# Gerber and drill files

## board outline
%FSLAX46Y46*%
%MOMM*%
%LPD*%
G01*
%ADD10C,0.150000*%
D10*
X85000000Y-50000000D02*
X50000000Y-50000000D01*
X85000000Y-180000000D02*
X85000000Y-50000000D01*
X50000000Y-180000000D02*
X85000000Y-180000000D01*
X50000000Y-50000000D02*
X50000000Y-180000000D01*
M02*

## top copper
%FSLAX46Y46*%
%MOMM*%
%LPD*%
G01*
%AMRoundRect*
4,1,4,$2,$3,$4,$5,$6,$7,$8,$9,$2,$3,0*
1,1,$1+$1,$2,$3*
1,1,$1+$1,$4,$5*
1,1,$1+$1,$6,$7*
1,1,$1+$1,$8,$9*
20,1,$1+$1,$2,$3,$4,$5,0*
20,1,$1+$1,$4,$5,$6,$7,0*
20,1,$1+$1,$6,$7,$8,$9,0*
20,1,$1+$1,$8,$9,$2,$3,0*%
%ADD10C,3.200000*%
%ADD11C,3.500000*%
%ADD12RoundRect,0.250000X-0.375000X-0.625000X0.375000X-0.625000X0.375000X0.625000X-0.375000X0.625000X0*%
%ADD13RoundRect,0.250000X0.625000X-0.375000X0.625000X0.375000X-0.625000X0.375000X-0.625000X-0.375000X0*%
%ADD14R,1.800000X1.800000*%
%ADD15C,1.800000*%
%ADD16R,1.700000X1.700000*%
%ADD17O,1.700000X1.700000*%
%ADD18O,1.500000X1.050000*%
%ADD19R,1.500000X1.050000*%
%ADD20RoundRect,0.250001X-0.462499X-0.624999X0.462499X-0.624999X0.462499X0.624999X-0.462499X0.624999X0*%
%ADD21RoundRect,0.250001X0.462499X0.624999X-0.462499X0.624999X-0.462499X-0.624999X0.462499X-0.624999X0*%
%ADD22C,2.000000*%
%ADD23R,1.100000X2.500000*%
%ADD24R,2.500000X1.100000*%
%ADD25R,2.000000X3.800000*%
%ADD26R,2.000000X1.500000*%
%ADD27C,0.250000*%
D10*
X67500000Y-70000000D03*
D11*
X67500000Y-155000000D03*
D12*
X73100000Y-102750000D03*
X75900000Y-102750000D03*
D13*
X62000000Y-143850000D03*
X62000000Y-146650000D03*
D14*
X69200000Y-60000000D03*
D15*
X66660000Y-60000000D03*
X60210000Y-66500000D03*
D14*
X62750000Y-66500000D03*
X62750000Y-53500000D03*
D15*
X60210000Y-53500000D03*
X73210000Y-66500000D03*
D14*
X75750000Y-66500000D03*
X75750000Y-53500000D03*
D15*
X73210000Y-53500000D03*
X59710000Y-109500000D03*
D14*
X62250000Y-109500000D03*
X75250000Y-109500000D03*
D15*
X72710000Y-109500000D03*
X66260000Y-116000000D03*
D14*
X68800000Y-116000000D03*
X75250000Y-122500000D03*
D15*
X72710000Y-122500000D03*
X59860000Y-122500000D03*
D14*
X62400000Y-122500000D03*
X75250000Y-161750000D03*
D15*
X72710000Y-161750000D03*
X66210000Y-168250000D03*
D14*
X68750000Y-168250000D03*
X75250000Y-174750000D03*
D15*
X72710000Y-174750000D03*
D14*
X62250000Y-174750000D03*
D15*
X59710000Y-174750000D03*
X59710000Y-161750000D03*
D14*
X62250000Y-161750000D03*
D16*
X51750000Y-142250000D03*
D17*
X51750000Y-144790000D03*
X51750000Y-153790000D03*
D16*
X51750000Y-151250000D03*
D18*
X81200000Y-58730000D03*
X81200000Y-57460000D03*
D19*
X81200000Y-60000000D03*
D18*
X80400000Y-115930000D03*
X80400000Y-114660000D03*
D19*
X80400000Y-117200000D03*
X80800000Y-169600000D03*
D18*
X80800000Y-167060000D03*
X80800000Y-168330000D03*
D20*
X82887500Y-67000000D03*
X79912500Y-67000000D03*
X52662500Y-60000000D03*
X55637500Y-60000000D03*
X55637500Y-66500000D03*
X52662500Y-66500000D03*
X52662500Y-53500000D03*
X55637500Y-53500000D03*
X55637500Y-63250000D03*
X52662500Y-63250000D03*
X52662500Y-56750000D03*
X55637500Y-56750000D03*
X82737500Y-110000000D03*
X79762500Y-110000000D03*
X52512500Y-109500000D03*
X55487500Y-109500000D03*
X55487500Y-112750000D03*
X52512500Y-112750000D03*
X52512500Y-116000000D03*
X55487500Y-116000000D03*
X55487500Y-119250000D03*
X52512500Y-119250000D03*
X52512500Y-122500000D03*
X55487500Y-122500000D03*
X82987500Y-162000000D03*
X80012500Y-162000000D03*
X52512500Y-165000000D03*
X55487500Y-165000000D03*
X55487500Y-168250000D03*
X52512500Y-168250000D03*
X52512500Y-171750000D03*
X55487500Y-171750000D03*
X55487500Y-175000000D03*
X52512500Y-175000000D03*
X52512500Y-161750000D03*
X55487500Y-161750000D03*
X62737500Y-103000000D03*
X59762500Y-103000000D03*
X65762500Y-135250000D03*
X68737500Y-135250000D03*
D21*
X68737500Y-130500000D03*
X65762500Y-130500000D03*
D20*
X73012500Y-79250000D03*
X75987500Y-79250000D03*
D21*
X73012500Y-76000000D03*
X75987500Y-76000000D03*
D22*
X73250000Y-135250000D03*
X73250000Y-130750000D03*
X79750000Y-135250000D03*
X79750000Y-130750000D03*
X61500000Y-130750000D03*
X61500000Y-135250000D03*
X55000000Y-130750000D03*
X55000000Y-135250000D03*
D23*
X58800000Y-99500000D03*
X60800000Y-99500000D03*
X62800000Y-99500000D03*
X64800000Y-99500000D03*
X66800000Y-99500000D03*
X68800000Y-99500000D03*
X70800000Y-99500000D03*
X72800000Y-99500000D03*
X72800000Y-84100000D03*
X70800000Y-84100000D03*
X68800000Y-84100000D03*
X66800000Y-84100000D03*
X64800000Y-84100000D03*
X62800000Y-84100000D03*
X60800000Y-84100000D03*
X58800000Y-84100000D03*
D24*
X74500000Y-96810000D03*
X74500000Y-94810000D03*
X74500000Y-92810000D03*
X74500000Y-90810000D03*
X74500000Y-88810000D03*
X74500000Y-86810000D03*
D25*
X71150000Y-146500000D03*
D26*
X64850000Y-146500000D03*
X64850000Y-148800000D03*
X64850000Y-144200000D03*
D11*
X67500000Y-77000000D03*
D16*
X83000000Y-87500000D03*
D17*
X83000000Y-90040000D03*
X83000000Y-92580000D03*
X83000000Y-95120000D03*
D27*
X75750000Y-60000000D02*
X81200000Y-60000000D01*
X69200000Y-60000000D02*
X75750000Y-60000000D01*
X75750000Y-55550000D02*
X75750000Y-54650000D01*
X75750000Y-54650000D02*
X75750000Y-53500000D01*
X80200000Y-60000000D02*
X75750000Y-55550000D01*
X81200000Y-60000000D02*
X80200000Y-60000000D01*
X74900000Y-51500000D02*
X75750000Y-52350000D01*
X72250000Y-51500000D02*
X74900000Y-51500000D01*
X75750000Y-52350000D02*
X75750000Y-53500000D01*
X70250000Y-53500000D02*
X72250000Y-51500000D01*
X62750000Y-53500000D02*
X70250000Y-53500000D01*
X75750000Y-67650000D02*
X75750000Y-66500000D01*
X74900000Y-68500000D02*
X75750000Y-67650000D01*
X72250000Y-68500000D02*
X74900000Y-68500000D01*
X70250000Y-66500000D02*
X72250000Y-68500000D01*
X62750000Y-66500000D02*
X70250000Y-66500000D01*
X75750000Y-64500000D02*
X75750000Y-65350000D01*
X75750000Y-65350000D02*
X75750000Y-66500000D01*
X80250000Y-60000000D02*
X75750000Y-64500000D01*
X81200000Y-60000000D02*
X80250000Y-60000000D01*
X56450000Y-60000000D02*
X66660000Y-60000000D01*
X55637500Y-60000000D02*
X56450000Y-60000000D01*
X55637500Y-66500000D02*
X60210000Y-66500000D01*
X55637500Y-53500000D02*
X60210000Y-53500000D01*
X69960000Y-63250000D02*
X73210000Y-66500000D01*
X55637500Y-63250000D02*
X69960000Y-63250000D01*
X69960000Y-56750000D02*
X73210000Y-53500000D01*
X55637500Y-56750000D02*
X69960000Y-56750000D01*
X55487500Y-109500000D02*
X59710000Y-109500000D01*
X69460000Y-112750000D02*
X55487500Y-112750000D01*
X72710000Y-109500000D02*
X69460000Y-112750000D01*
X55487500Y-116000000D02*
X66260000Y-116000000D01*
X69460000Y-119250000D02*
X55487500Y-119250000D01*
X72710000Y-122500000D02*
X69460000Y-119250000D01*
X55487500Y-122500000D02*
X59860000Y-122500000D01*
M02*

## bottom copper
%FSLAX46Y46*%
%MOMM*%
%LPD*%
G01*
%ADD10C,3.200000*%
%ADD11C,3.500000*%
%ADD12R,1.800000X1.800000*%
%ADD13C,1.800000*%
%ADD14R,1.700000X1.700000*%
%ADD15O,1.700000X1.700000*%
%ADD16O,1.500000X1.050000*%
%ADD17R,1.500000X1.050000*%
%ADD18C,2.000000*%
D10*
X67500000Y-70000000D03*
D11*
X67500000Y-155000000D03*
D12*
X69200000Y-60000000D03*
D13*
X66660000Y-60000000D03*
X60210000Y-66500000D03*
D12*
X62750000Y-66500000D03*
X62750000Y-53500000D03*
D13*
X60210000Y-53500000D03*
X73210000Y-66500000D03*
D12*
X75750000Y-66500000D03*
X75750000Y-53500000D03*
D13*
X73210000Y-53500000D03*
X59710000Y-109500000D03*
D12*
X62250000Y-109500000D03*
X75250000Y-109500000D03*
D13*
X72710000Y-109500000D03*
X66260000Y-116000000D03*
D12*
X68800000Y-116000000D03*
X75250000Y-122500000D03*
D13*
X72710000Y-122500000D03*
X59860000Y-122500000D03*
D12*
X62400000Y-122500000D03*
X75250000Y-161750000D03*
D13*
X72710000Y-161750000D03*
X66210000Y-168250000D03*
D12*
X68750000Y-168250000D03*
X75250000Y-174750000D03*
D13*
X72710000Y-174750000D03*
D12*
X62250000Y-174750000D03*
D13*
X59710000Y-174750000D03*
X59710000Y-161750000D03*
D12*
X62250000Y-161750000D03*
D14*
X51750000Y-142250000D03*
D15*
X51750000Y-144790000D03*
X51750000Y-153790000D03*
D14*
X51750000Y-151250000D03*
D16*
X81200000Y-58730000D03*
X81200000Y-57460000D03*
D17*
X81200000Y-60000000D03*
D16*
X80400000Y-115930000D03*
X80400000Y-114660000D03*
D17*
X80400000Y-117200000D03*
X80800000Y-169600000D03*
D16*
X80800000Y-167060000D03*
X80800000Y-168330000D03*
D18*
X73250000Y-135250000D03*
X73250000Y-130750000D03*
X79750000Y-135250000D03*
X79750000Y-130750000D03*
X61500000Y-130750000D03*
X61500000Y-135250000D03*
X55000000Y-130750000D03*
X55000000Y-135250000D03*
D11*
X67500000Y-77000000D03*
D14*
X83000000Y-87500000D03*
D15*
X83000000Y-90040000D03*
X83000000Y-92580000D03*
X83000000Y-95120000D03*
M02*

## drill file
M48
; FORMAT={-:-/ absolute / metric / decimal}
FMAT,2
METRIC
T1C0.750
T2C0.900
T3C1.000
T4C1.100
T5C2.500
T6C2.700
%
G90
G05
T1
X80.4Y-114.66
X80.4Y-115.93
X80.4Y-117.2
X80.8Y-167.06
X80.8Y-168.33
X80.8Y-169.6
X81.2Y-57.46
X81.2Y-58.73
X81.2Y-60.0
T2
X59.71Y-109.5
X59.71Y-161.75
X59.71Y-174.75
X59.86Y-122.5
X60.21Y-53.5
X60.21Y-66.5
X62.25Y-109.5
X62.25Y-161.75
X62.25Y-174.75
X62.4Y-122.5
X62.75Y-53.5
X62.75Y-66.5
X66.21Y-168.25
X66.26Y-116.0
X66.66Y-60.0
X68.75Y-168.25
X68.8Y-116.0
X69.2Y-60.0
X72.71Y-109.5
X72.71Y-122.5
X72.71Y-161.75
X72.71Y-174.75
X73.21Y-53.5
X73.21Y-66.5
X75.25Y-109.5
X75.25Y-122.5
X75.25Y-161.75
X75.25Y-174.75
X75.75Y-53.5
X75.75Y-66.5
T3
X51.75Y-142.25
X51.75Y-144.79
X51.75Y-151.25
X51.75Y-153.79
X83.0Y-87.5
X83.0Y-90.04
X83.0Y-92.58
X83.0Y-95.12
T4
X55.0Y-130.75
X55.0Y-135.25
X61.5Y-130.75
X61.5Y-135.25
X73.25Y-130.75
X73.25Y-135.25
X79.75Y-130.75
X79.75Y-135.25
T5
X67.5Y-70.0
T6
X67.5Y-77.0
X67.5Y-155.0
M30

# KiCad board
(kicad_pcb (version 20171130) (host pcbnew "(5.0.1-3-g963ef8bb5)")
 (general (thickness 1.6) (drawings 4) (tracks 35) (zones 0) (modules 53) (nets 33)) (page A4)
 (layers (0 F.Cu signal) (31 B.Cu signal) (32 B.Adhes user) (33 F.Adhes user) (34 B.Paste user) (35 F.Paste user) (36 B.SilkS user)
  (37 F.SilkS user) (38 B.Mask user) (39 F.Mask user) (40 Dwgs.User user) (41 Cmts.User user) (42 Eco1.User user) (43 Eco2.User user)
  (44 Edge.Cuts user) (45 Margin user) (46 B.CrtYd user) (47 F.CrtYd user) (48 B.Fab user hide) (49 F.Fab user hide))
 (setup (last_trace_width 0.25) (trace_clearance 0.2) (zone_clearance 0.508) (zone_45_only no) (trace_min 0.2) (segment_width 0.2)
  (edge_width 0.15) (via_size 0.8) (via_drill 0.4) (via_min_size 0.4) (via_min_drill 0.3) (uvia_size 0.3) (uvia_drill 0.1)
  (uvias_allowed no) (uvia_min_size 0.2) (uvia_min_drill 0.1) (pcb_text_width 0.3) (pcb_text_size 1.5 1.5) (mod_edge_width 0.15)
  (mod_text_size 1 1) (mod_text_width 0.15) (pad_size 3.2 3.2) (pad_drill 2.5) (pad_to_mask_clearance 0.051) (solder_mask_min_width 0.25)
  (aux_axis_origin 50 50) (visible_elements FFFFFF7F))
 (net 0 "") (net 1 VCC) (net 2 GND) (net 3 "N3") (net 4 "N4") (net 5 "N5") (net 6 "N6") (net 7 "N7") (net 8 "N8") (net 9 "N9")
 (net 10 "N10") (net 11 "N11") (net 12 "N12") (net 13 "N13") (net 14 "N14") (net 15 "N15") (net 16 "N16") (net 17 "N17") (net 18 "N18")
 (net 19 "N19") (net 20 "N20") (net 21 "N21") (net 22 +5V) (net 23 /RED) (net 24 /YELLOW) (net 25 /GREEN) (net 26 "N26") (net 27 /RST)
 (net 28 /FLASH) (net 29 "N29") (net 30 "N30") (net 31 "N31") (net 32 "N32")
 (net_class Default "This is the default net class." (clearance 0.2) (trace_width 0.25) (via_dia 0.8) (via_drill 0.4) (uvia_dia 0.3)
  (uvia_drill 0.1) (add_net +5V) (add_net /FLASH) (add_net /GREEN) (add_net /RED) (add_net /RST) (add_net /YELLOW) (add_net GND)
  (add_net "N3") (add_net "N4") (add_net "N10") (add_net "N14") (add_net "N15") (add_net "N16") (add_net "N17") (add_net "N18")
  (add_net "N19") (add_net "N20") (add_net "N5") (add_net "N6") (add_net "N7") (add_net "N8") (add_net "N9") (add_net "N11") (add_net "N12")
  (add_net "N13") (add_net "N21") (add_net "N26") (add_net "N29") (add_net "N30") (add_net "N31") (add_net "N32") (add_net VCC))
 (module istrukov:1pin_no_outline (layer F.Cu) (at 67.8 70)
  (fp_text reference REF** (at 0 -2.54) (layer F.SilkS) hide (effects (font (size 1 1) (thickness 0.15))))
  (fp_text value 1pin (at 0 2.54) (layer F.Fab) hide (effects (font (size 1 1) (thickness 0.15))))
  (pad "" thru_hole circle (at -0.3 0) (size 3.2 3.2) (drill 2.5) (layers *.Cu *.Mask)))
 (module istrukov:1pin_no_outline (layer F.Cu) (at 67.5 155)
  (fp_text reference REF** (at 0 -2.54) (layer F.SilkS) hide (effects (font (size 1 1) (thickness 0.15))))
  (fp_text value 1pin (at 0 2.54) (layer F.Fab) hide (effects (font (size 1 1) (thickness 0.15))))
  (pad "" thru_hole circle (at 0 0) (size 3.5 3.5) (drill 2.7) (layers *.Cu *.Mask)))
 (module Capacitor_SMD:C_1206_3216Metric (layer F.Cu) (at 74.5 102.75)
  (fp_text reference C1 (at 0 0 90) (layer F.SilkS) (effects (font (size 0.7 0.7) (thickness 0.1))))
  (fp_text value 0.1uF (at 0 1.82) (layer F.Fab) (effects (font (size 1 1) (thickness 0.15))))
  (pad 1 smd roundrect (at -1.4 0) (size 1.25 1.75) (layers F.Cu F.Paste F.Mask) (roundrect_rratio 0.2) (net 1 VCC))
  (pad 2 smd roundrect (at 1.4 0) (size 1.25 1.75) (layers F.Cu F.Paste F.Mask) (roundrect_rratio 0.2) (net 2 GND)))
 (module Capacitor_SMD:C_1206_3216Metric (layer F.Cu) (at 62 145.25 90)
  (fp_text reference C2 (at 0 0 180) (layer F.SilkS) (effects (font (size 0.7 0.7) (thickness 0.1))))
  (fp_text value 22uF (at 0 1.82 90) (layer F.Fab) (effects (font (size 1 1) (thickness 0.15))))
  (pad 2 smd roundrect (at 1.4 0 90) (size 1.25 1.75) (layers F.Cu F.Paste F.Mask) (roundrect_rratio 0.2) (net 2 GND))
  (pad 1 smd roundrect (at -1.4 0 90) (size 1.25 1.75) (layers F.Cu F.Paste F.Mask) (roundrect_rratio 0.2) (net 1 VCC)))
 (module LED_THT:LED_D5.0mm (layer F.Cu) (at 69.2 60 180)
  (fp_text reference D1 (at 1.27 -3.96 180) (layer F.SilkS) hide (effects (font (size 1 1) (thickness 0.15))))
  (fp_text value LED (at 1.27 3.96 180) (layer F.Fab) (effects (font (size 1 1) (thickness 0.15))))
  (pad 1 thru_hole rect (at 0 0 180) (size 1.8 1.8) (drill 0.9) (layers *.Cu *.Mask) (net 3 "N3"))
  (pad 2 thru_hole circle (at 2.54 0 180) (size 1.8 1.8) (drill 0.9) (layers *.Cu *.Mask) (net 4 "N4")))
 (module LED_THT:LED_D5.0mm (layer F.Cu) (at 62.75 66.5 180)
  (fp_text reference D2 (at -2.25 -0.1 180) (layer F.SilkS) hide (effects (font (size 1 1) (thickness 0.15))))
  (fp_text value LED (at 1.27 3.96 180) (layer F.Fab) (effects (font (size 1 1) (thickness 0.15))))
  (pad 2 thru_hole circle (at 2.54 0 180) (size 1.8 1.8) (drill 0.9) (layers *.Cu *.Mask) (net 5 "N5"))
  (pad 1 thru_hole rect (at 0 0 180) (size 1.8 1.8) (drill 0.9) (layers *.Cu *.Mask) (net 3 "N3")))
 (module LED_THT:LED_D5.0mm (layer F.Cu) (at 62.75 53.5 180)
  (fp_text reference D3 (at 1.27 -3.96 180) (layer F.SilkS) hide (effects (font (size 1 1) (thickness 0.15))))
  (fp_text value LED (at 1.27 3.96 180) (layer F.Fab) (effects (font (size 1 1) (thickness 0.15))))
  (pad 1 thru_hole rect (at 0 0 180) (size 1.8 1.8) (drill 0.9) (layers *.Cu *.Mask) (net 3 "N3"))
  (pad 2 thru_hole circle (at 2.54 0 180) (size 1.8 1.8) (drill 0.9) (layers *.Cu *.Mask) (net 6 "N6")))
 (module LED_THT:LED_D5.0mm (layer F.Cu) (at 75.75 66.5 180)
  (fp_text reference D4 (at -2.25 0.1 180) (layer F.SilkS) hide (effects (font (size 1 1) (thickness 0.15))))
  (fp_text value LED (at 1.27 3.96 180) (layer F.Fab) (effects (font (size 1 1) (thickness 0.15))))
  (pad 2 thru_hole circle (at 2.54 0 180) (size 1.8 1.8) (drill 0.9) (layers *.Cu *.Mask) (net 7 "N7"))
  (pad 1 thru_hole rect (at 0 0 180) (size 1.8 1.8) (drill 0.9) (layers *.Cu *.Mask) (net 3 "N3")))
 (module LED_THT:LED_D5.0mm (layer F.Cu) (at 75.75 53.5 180)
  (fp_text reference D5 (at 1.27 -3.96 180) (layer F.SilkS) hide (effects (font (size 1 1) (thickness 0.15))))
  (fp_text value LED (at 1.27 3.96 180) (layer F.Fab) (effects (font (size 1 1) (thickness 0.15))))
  (pad 1 thru_hole rect (at 0 0 180) (size 1.8 1.8) (drill 0.9) (layers *.Cu *.Mask) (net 3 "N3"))
  (pad 2 thru_hole circle (at 2.54 0 180) (size 1.8 1.8) (drill 0.9) (layers *.Cu *.Mask) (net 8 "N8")))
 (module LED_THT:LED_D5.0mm (layer F.Cu) (at 62.25 109.5 180)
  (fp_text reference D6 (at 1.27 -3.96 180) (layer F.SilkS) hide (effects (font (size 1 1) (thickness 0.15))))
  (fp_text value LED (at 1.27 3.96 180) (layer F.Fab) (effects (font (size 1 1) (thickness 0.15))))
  (pad 2 thru_hole circle (at 2.54 0 180) (size 1.8 1.8) (drill 0.9) (layers *.Cu *.Mask) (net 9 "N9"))
  (pad 1 thru_hole rect (at 0 0 180) (size 1.8 1.8) (drill 0.9) (layers *.Cu *.Mask) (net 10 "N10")))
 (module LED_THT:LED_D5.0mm (layer F.Cu) (at 75.25 109.5 180)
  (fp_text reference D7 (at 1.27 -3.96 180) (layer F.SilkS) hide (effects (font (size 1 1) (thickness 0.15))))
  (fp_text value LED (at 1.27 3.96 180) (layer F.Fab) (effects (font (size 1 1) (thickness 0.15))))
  (pad 1 thru_hole rect (at 0 0 180) (size 1.8 1.8) (drill 0.9) (layers *.Cu *.Mask) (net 10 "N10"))
  (pad 2 thru_hole circle (at 2.54 0 180) (size 1.8 1.8) (drill 0.9) (layers *.Cu *.Mask) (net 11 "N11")))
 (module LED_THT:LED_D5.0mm (layer F.Cu) (at 68.8 116 180)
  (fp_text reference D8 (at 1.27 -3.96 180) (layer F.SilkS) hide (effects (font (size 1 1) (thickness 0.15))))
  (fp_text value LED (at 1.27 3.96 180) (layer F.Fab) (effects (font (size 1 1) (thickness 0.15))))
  (pad 2 thru_hole circle (at 2.54 0 180) (size 1.8 1.8) (drill 0.9) (layers *.Cu *.Mask) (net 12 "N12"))
  (pad 1 thru_hole rect (at 0 0 180) (size 1.8 1.8) (drill 0.9) (layers *.Cu *.Mask) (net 10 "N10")))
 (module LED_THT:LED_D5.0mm (layer F.Cu) (at 75.25 122.5 180)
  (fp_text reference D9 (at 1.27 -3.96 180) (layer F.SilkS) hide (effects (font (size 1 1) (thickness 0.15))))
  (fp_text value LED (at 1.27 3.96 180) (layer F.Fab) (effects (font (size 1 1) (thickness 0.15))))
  (pad 1 thru_hole rect (at 0 0 180) (size 1.8 1.8) (drill 0.9) (layers *.Cu *.Mask) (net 10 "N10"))
  (pad 2 thru_hole circle (at 2.54 0 180) (size 1.8 1.8) (drill 0.9) (layers *.Cu *.Mask) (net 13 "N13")))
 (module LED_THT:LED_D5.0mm (layer F.Cu) (at 62.4 122.5 180)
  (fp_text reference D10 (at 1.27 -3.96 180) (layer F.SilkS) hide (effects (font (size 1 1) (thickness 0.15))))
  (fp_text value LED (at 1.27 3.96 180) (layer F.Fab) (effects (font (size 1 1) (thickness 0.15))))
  (pad 2 thru_hole circle (at 2.54 0 180) (size 1.8 1.8) (drill 0.9) (layers *.Cu *.Mask) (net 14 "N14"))
  (pad 1 thru_hole rect (at 0 0 180) (size 1.8 1.8) (drill 0.9) (layers *.Cu *.Mask) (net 10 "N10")))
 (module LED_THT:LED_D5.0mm (layer F.Cu) (at 75.25 161.75 180)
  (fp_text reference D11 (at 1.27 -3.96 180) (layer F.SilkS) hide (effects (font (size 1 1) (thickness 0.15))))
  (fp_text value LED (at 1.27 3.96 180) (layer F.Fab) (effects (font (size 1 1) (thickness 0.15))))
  (pad 1 thru_hole rect (at 0 0 180) (size 1.8 1.8) (drill 0.9) (layers *.Cu *.Mask) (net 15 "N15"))
  (pad 2 thru_hole circle (at 2.54 0 180) (size 1.8 1.8) (drill 0.9) (layers *.Cu *.Mask) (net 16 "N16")))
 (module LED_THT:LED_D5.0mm (layer F.Cu) (at 68.75 168.25 180)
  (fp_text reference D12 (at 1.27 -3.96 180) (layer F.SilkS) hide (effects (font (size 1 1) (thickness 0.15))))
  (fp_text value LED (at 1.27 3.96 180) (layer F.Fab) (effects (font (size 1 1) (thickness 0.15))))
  (pad 2 thru_hole circle (at 2.54 0 180) (size 1.8 1.8) (drill 0.9) (layers *.Cu *.Mask) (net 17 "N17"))
  (pad 1 thru_hole rect (at 0 0 180) (size 1.8 1.8) (drill 0.9) (layers *.Cu *.Mask) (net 15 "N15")))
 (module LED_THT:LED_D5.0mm (layer F.Cu) (at 75.25 174.75 180)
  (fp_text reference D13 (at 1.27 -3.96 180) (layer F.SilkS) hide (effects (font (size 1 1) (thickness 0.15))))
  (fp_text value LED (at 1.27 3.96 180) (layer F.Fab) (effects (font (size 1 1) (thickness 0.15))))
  (pad 1 thru_hole rect (at 0 0 180) (size 1.8 1.8) (drill 0.9) (layers *.Cu *.Mask) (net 15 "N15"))
  (pad 2 thru_hole circle (at 2.54 0 180) (size 1.8 1.8) (drill 0.9) (layers *.Cu *.Mask) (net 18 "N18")))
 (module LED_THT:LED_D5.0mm (layer F.Cu) (at 62.25 174.75 180)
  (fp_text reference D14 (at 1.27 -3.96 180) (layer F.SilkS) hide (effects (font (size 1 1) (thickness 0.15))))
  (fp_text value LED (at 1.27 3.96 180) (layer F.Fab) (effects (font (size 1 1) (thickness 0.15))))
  (pad 1 thru_hole rect (at 0 0 180) (size 1.8 1.8) (drill 0.9) (layers *.Cu *.Mask) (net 15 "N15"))
  (pad 2 thru_hole circle (at 2.54 0 180) (size 1.8 1.8) (drill 0.9) (layers *.Cu *.Mask) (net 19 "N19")))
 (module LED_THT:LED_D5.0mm (layer F.Cu) (at 62.25 161.75 180)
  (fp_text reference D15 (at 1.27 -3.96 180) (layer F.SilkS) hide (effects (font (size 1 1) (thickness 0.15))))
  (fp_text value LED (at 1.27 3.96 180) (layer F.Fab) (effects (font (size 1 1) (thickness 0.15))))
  (pad 2 thru_hole circle (at 2.54 0 180) (size 1.8 1.8) (drill 0.9) (layers *.Cu *.Mask) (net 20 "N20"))
  (pad 1 thru_hole rect (at 0 0 180) (size 1.8 1.8) (drill 0.9) (layers *.Cu *.Mask) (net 15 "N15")))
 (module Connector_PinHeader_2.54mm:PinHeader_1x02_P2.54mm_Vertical (layer F.Cu) (at 51.75 142.25)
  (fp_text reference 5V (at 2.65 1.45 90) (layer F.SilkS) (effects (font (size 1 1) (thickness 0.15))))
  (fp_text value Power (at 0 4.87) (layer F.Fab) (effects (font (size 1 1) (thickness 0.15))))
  (pad 1 thru_hole rect (at 0 0) (size 1.7 1.7) (drill 1) (layers *.Cu *.Mask) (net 2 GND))
  (pad 2 thru_hole oval (at 0 2.54) (size 1.7 1.7) (drill 1) (layers *.Cu *.Mask) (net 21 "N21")))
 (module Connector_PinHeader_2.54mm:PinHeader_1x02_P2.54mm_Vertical (layer F.Cu) (at 51.75 151.25)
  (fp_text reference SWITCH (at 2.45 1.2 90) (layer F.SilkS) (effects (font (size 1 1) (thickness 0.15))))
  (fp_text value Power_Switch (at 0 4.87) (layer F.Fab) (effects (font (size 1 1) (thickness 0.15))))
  (pad 2 thru_hole oval (at 0 2.54) (size 1.7 1.7) (drill 1) (layers *.Cu *.Mask) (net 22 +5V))
  (pad 1 thru_hole rect (at 0 0) (size 1.7 1.7) (drill 1) (layers *.Cu *.Mask) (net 21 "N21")))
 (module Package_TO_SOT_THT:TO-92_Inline (layer F.Cu) (at 81.2 60 90)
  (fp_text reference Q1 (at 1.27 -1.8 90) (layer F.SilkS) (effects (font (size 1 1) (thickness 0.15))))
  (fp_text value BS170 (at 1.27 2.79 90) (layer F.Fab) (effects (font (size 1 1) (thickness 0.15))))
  (pad 2 thru_hole oval (at 1.27 0 90) (size 1.05 1.5) (drill 0.75) (layers *.Cu *.Mask) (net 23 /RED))
  (pad 3 thru_hole oval (at 2.54 0 90) (size 1.05 1.5) (drill 0.75) (layers *.Cu *.Mask) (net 2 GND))
  (pad 1 thru_hole rect (at 0 0 90) (size 1.05 1.5) (drill 0.75) (layers *.Cu *.Mask) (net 3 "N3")))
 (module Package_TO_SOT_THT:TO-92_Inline (layer F.Cu) (at 80.4 117.2 90)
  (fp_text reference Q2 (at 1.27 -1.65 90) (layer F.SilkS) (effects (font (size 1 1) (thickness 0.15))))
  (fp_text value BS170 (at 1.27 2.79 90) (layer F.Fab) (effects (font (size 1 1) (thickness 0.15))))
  (pad 2 thru_hole oval (at 1.27 0 90) (size 1.05 1.5) (drill 0.75) (layers *.Cu *.Mask) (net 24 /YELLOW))
  (pad 3 thru_hole oval (at 2.54 0 90) (size 1.05 1.5) (drill 0.75) (layers *.Cu *.Mask) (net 2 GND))
  (pad 1 thru_hole rect (at 0 0 90) (size 1.05 1.5) (drill 0.75) (layers *.Cu *.Mask) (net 10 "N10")))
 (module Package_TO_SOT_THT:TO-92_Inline (layer F.Cu) (at 80.8 169.6 90)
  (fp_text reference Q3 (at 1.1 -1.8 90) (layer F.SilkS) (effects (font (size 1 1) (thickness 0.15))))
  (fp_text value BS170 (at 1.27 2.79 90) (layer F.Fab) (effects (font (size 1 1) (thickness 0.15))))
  (pad 1 thru_hole rect (at 0 0 90) (size 1.05 1.5) (drill 0.75) (layers *.Cu *.Mask) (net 15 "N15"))
  (pad 3 thru_hole oval (at 2.54 0 90) (size 1.05 1.5) (drill 0.75) (layers *.Cu *.Mask) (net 2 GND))
  (pad 2 thru_hole oval (at 1.27 0 90) (size 1.05 1.5) (drill 0.75) (layers *.Cu *.Mask) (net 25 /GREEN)))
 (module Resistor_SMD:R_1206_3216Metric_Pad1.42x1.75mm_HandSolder (layer F.Cu) (at 81.4 67)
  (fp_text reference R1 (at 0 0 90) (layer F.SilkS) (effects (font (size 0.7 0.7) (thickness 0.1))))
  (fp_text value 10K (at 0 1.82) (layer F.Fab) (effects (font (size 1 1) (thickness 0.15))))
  (pad 2 smd roundrect (at 1.4875 0) (size 1.425 1.75) (layers F.Cu F.Paste F.Mask) (roundrect_rratio 0.175439) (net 2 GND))
  (pad 1 smd roundrect (at -1.4875 0) (size 1.425 1.75) (layers F.Cu F.Paste F.Mask) (roundrect_rratio 0.175439) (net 23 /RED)))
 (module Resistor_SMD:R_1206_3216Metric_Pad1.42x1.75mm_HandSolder (layer F.Cu) (at 54.15 60)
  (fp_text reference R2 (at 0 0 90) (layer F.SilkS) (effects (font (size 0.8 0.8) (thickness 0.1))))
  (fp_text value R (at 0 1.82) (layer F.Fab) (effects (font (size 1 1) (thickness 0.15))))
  (pad 1 smd roundrect (at -1.4875 0) (size 1.425 1.75) (layers F.Cu F.Paste F.Mask) (roundrect_rratio 0.175439) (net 22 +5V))
  (pad 2 smd roundrect (at 1.4875 0) (size 1.425 1.75) (layers F.Cu F.Paste F.Mask) (roundrect_rratio 0.175439) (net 4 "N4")))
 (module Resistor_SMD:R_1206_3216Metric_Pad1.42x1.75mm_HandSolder (layer F.Cu) (at 54.15 66.5)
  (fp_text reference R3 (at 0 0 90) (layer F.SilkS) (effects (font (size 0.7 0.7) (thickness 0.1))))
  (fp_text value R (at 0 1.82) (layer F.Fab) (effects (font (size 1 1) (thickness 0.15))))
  (pad 2 smd roundrect (at 1.4875 0) (size 1.425 1.75) (layers F.Cu F.Paste F.Mask) (roundrect_rratio 0.175439) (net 5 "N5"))
  (pad 1 smd roundrect (at -1.4875 0) (size 1.425 1.75) (layers F.Cu F.Paste F.Mask) (roundrect_rratio 0.175439) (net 22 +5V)))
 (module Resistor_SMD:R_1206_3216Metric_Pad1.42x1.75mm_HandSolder (layer F.Cu) (at 54.15 53.5)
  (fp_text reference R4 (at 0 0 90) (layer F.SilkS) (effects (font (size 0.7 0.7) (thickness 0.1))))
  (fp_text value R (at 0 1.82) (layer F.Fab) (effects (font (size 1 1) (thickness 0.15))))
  (pad 1 smd roundrect (at -1.4875 0) (size 1.425 1.75) (layers F.Cu F.Paste F.Mask) (roundrect_rratio 0.175439) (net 22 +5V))
  (pad 2 smd roundrect (at 1.4875 0) (size 1.425 1.75) (layers F.Cu F.Paste F.Mask) (roundrect_rratio 0.175439) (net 6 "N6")))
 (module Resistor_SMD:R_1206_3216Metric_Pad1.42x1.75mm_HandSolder (layer F.Cu) (at 54.15 63.25)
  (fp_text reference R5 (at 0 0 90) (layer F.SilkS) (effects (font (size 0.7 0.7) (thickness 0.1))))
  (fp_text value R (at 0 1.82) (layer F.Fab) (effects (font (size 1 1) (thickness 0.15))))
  (pad 2 smd roundrect (at 1.4875 0) (size 1.425 1.75) (layers F.Cu F.Paste F.Mask) (roundrect_rratio 0.175439) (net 7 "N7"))
  (pad 1 smd roundrect (at -1.4875 0) (size 1.425 1.75) (layers F.Cu F.Paste F.Mask) (roundrect_rratio 0.175439) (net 22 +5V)))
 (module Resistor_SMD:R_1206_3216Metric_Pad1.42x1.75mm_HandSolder (layer F.Cu) (at 54.15 56.75)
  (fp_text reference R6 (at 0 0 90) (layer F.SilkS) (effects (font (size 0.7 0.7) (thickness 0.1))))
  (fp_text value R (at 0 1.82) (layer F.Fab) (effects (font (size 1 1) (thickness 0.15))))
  (pad 1 smd roundrect (at -1.4875 0) (size 1.425 1.75) (layers F.Cu F.Paste F.Mask) (roundrect_rratio 0.175439) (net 22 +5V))
  (pad 2 smd roundrect (at 1.4875 0) (size 1.425 1.75) (layers F.Cu F.Paste F.Mask) (roundrect_rratio 0.175439) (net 8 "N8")))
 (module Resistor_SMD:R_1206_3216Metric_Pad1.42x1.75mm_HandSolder (layer F.Cu) (at 81.25 110)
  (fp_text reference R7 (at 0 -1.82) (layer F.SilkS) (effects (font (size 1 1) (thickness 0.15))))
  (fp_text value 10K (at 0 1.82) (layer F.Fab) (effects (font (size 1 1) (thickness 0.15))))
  (pad 2 smd roundrect (at 1.4875 0) (size 1.425 1.75) (layers F.Cu F.Paste F.Mask) (roundrect_rratio 0.175439) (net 2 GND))
  (pad 1 smd roundrect (at -1.4875 0) (size 1.425 1.75) (layers F.Cu F.Paste F.Mask) (roundrect_rratio 0.175439) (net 24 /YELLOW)))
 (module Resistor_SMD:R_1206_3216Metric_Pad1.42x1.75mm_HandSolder (layer F.Cu) (at 54 109.5)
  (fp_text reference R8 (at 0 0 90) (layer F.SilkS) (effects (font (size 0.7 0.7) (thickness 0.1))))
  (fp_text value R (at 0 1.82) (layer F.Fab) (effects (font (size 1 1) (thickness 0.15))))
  (pad 1 smd roundrect (at -1.4875 0) (size 1.425 1.75) (layers F.Cu F.Paste F.Mask) (roundrect_rratio 0.175439) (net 22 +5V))
  (pad 2 smd roundrect (at 1.4875 0) (size 1.425 1.75) (layers F.Cu F.Paste F.Mask) (roundrect_rratio 0.175439) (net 9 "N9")))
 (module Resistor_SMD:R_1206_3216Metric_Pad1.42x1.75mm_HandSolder (layer F.Cu) (at 54 112.75)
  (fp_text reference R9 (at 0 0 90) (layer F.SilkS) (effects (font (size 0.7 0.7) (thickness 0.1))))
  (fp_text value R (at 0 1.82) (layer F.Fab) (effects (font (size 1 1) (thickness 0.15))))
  (pad 2 smd roundrect (at 1.4875 0) (size 1.425 1.75) (layers F.Cu F.Paste F.Mask) (roundrect_rratio 0.175439) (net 11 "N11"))
  (pad 1 smd roundrect (at -1.4875 0) (size 1.425 1.75) (layers F.Cu F.Paste F.Mask) (roundrect_rratio 0.175439) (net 22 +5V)))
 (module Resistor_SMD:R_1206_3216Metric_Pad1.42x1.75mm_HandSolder (layer F.Cu) (at 54 116)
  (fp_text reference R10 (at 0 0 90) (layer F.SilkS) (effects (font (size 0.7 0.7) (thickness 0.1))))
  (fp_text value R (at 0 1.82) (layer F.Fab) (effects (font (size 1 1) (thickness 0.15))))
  (pad 1 smd roundrect (at -1.4875 0) (size 1.425 1.75) (layers F.Cu F.Paste F.Mask) (roundrect_rratio 0.175439) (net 22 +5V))
  (pad 2 smd roundrect (at 1.4875 0) (size 1.425 1.75) (layers F.Cu F.Paste F.Mask) (roundrect_rratio 0.175439) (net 12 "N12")))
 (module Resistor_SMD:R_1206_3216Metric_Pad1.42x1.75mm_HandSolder (layer F.Cu) (at 54 119.25)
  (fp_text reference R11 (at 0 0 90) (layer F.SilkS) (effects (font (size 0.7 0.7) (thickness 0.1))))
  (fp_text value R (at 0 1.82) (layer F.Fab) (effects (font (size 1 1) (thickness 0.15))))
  (pad 2 smd roundrect (at 1.4875 0) (size 1.425 1.75) (layers F.Cu F.Paste F.Mask) (roundrect_rratio 0.175439) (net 13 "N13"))
  (pad 1 smd roundrect (at -1.4875 0) (size 1.425 1.75) (layers F.Cu F.Paste F.Mask) (roundrect_rratio 0.175439) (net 22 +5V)))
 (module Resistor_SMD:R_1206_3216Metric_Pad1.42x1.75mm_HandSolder (layer F.Cu) (at 54 122.5)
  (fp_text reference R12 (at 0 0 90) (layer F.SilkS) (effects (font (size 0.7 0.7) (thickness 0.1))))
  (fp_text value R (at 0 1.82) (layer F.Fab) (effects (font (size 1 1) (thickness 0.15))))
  (pad 1 smd roundrect (at -1.4875 0) (size 1.425 1.75) (layers F.Cu F.Paste F.Mask) (roundrect_rratio 0.175439) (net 22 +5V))
  (pad 2 smd roundrect (at 1.4875 0) (size 1.425 1.75) (layers F.Cu F.Paste F.Mask) (roundrect_rratio 0.175439) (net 14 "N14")))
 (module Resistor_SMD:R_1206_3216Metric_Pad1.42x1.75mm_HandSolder (layer F.Cu) (at 81.5 162)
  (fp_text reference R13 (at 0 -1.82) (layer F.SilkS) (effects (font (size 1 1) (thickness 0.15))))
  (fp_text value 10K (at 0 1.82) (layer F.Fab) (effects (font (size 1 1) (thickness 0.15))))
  (pad 2 smd roundrect (at 1.4875 0) (size 1.425 1.75) (layers F.Cu F.Paste F.Mask) (roundrect_rratio 0.175439) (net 2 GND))
  (pad 1 smd roundrect (at -1.4875 0) (size 1.425 1.75) (layers F.Cu F.Paste F.Mask) (roundrect_rratio 0.175439) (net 25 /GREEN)))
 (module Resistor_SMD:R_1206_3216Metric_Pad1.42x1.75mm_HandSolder (layer F.Cu) (at 54 165)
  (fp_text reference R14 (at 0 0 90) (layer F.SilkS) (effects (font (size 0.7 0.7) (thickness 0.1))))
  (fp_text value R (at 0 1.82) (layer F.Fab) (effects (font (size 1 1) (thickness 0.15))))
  (pad 1 smd roundrect (at -1.4875 0) (size 1.425 1.75) (layers F.Cu F.Paste F.Mask) (roundrect_rratio 0.175439) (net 22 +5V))
  (pad 2 smd roundrect (at 1.4875 0) (size 1.425 1.75) (layers F.Cu F.Paste F.Mask) (roundrect_rratio 0.175439) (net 16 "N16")))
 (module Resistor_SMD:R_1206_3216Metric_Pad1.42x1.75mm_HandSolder (layer F.Cu) (at 54 168.25)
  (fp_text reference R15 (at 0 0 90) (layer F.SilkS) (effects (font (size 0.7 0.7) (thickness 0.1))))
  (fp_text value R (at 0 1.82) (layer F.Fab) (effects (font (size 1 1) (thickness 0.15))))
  (pad 2 smd roundrect (at 1.4875 0) (size 1.425 1.75) (layers F.Cu F.Paste F.Mask) (roundrect_rratio 0.175439) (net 17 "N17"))
  (pad 1 smd roundrect (at -1.4875 0) (size 1.425 1.75) (layers F.Cu F.Paste F.Mask) (roundrect_rratio 0.175439) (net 22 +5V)))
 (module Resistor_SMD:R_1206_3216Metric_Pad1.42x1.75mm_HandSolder (layer F.Cu) (at 54 171.75)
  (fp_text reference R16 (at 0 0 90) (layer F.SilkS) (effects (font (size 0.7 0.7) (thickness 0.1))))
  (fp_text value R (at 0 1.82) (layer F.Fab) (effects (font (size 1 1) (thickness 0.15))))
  (pad 1 smd roundrect (at -1.4875 0) (size 1.425 1.75) (layers F.Cu F.Paste F.Mask) (roundrect_rratio 0.175439) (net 22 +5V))
  (pad 2 smd roundrect (at 1.4875 0) (size 1.425 1.75) (layers F.Cu F.Paste F.Mask) (roundrect_rratio 0.175439) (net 18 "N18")))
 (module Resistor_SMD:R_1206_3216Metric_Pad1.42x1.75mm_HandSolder (layer F.Cu) (at 54 175)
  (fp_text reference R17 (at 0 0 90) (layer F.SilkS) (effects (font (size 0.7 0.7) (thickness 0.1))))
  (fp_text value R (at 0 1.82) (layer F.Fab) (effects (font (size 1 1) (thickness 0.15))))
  (pad 2 smd roundrect (at 1.4875 0) (size 1.425 1.75) (layers F.Cu F.Paste F.Mask) (roundrect_rratio 0.175439) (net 19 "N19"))
  (pad 1 smd roundrect (at -1.4875 0) (size 1.425 1.75) (layers F.Cu F.Paste F.Mask) (roundrect_rratio 0.175439) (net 22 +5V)))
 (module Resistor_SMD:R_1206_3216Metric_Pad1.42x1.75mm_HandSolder (layer F.Cu) (at 54 161.75)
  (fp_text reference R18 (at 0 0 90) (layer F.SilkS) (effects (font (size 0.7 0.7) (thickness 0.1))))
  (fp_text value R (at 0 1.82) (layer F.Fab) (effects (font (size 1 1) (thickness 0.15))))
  (pad 1 smd roundrect (at -1.4875 0) (size 1.425 1.75) (layers F.Cu F.Paste F.Mask) (roundrect_rratio 0.175439) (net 22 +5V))
  (pad 2 smd roundrect (at 1.4875 0) (size 1.425 1.75) (layers F.Cu F.Paste F.Mask) (roundrect_rratio 0.175439) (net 20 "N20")))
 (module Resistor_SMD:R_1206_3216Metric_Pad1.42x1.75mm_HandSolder (layer F.Cu) (at 61.25 103)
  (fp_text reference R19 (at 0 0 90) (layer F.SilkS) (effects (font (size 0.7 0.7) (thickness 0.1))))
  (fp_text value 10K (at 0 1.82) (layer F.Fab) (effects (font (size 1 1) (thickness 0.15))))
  (pad 2 smd roundrect (at 1.4875 0) (size 1.425 1.75) (layers F.Cu F.Paste F.Mask) (roundrect_rratio 0.175439) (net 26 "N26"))
  (pad 1 smd roundrect (at -1.4875 0) (size 1.425 1.75) (layers F.Cu F.Paste F.Mask) (roundrect_rratio 0.175439) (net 1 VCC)))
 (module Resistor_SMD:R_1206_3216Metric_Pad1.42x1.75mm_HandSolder (layer F.Cu) (at 67.25 135.25)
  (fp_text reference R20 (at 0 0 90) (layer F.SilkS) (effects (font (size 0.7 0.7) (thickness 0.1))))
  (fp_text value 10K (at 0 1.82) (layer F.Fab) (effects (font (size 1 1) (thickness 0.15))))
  (pad 1 smd roundrect (at -1.4875 0) (size 1.425 1.75) (layers F.Cu F.Paste F.Mask) (roundrect_rratio 0.175439) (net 1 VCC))
  (pad 2 smd roundrect (at 1.4875 0) (size 1.425 1.75) (layers F.Cu F.Paste F.Mask) (roundrect_rratio 0.175439) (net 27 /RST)))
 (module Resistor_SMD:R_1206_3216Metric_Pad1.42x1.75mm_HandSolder (layer F.Cu) (at 67.25 130.5 180)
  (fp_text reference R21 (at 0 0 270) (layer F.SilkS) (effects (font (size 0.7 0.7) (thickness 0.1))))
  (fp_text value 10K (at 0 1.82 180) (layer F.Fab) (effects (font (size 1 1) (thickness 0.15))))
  (pad 1 smd roundrect (at -1.4875 0 180) (size 1.425 1.75) (layers F.Cu F.Paste F.Mask) (roundrect_rratio 0.175439) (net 1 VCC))
  (pad 2 smd roundrect (at 1.4875 0 180) (size 1.425 1.75) (layers F.Cu F.Paste F.Mask) (roundrect_rratio 0.175439) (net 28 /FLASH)))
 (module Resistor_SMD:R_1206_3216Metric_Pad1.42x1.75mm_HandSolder (layer F.Cu) (at 74.5 79.25)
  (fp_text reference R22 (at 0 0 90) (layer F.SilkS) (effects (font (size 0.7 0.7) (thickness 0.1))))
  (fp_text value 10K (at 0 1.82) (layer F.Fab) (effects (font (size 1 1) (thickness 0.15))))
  (pad 1 smd roundrect (at -1.4875 0) (size 1.425 1.75) (layers F.Cu F.Paste F.Mask) (roundrect_rratio 0.175439) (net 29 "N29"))
  (pad 2 smd roundrect (at 1.4875 0) (size 1.425 1.75) (layers F.Cu F.Paste F.Mask) (roundrect_rratio 0.175439) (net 2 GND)))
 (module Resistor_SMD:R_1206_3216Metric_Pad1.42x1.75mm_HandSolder (layer F.Cu) (at 74.5 76 180)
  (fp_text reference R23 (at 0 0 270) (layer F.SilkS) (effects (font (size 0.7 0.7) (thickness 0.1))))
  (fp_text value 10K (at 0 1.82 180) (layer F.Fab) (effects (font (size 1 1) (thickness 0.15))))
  (pad 2 smd roundrect (at 1.4875 0 180) (size 1.425 1.75) (layers F.Cu F.Paste F.Mask) (roundrect_rratio 0.175439) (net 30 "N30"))
  (pad 1 smd roundrect (at -1.4875 0 180) (size 1.425 1.75) (layers F.Cu F.Paste F.Mask) (roundrect_rratio 0.175439) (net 1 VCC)))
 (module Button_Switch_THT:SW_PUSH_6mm (layer F.Cu) (at 79.75 135.25 180)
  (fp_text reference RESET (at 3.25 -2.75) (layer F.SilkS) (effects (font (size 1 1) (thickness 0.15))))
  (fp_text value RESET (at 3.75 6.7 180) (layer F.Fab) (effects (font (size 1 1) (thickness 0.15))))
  (pad 1 thru_hole circle (at 6.5 0 270) (size 2 2) (drill 1.1) (layers *.Cu *.Mask) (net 27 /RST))
  (pad 2 thru_hole circle (at 6.5 4.5 270) (size 2 2) (drill 1.1) (layers *.Cu *.Mask) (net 2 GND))
  (pad 1 thru_hole circle (at 0 0 270) (size 2 2) (drill 1.1) (layers *.Cu *.Mask) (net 27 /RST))
  (pad 2 thru_hole circle (at 0 4.5 270) (size 2 2) (drill 1.1) (layers *.Cu *.Mask) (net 2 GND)))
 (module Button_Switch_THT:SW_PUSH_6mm (layer F.Cu) (at 61.5 135.25 180)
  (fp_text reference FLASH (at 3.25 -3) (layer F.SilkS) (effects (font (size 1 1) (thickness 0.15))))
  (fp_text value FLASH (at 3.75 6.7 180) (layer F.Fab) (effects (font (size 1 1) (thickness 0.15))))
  (pad 2 thru_hole circle (at 0 4.5 270) (size 2 2) (drill 1.1) (layers *.Cu *.Mask) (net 2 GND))
  (pad 1 thru_hole circle (at 0 0 270) (size 2 2) (drill 1.1) (layers *.Cu *.Mask) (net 28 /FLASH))
  (pad 2 thru_hole circle (at 6.5 4.5 270) (size 2 2) (drill 1.1) (layers *.Cu *.Mask) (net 2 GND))
  (pad 1 thru_hole circle (at 6.5 0 270) (size 2 2) (drill 1.1) (layers *.Cu *.Mask) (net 28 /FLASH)))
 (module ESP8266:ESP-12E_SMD (layer F.Cu) (at 58.8 98.8 90)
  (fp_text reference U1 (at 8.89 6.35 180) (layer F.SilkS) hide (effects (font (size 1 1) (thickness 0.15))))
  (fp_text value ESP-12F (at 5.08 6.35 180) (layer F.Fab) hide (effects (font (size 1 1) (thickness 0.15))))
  (pad 1 smd rect (at 0 0 90) (size 2.5 1.1) (drill (offset -0.7 0)) (layers F.Cu F.Paste F.Mask) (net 27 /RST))
  (pad 2 smd rect (at 0 2 90) (size 2.5 1.1) (drill (offset -0.7 0)) (layers F.Cu F.Paste F.Mask))
  (pad 3 smd rect (at 0 4 90) (size 2.5 1.1) (drill (offset -0.7 0)) (layers F.Cu F.Paste F.Mask) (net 26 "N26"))
  (pad 4 smd rect (at 0 6 90) (size 2.5 1.1) (drill (offset -0.7 0)) (layers F.Cu F.Paste F.Mask))
  (pad 5 smd rect (at 0 8 90) (size 2.5 1.1) (drill (offset -0.7 0)) (layers F.Cu F.Paste F.Mask) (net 25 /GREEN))
  (pad 6 smd rect (at 0 10 90) (size 2.5 1.1) (drill (offset -0.7 0)) (layers F.Cu F.Paste F.Mask) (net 23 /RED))
  (pad 7 smd rect (at 0 12 90) (size 2.5 1.1) (drill (offset -0.7 0)) (layers F.Cu F.Paste F.Mask) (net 24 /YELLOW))
  (pad 8 smd rect (at 0 14 90) (size 2.5 1.1) (drill (offset -0.7 0)) (layers F.Cu F.Paste F.Mask) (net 1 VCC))
  (pad 9 smd rect (at 14 14 90) (size 2.5 1.1) (drill (offset 0.7 0)) (layers F.Cu F.Paste F.Mask) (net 2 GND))
  (pad 10 smd rect (at 14 12 90) (size 2.5 1.1) (drill (offset 0.7 0)) (layers F.Cu F.Paste F.Mask) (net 29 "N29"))
  (pad 11 smd rect (at 14 10 90) (size 2.5 1.1) (drill (offset 0.7 0)) (layers F.Cu F.Paste F.Mask) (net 30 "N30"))
  (pad 12 smd rect (at 14 8 90) (size 2.5 1.1) (drill (offset 0.7 0)) (layers F.Cu F.Paste F.Mask) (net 28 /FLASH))
  (pad 13 smd rect (at 14 6 90) (size 2.5 1.1) (drill (offset 0.7 0)) (layers F.Cu F.Paste F.Mask))
  (pad 14 smd rect (at 14 4 90) (size 2.5 1.1) (drill (offset 0.7 0)) (layers F.Cu F.Paste F.Mask))
  (pad 15 smd rect (at 14 2 90) (size 2.5 1.1) (drill (offset 0.7 0)) (layers F.Cu F.Paste F.Mask) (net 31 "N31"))
  (pad 16 smd rect (at 14 0 90) (size 2.5 1.1) (drill (offset 0.7 0)) (layers F.Cu F.Paste F.Mask) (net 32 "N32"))
  (pad 17 smd rect (at 1.99 15 180) (size 2.5 1.1) (drill (offset -0.7 0)) (layers F.Cu F.Paste F.Mask))
  (pad 18 smd rect (at 3.99 15 180) (size 2.5 1.1) (drill (offset -0.7 0)) (layers F.Cu F.Paste F.Mask))
  (pad 19 smd rect (at 5.99 15 180) (size 2.5 1.1) (drill (offset -0.7 0)) (layers F.Cu F.Paste F.Mask))
  (pad 20 smd rect (at 7.99 15 180) (size 2.5 1.1) (drill (offset -0.7 0)) (layers F.Cu F.Paste F.Mask))
  (pad 21 smd rect (at 9.99 15 180) (size 2.5 1.1) (drill (offset -0.7 0)) (layers F.Cu F.Paste F.Mask))
  (pad 22 smd rect (at 11.99 15 180) (size 2.5 1.1) (drill (offset -0.7 0)) (layers F.Cu F.Paste F.Mask)))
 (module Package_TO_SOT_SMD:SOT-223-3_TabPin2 (layer F.Cu) (at 68 146.5)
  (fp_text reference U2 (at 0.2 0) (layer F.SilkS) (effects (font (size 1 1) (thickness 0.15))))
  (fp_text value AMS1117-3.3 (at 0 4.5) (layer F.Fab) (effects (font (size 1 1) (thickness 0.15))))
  (pad 2 smd rect (at 3.15 0) (size 2 3.8) (layers F.Cu F.Paste F.Mask) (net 1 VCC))
  (pad 2 smd rect (at -3.15 0) (size 2 1.5) (layers F.Cu F.Paste F.Mask) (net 1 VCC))
  (pad 3 smd rect (at -3.15 2.3) (size 2 1.5) (layers F.Cu F.Paste F.Mask) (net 22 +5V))
  (pad 1 smd rect (at -3.15 -2.3) (size 2 1.5) (layers F.Cu F.Paste F.Mask) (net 2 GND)))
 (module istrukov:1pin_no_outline (layer F.Cu) (at 67.5 77)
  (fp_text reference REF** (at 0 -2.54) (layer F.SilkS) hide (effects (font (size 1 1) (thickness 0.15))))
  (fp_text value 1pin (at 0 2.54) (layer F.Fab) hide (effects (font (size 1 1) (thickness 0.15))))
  (pad "" thru_hole circle (at 0 0) (size 3.5 3.5) (drill 2.7) (layers *.Cu *.Mask)))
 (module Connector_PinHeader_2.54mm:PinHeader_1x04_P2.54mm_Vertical (layer F.Cu) (at 83 87.5)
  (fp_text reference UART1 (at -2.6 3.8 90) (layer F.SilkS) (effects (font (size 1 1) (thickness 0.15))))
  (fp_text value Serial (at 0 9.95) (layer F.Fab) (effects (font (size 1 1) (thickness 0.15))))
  (pad 1 thru_hole rect (at 0 0) (size 1.7 1.7) (drill 1) (layers *.Cu *.Mask) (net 1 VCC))
  (pad 2 thru_hole oval (at 0 2.54) (size 1.7 1.7) (drill 1) (layers *.Cu *.Mask) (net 2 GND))
  (pad 3 thru_hole oval (at 0 5.08) (size 1.7 1.7) (drill 1) (layers *.Cu *.Mask) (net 32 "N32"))
  (pad 4 thru_hole oval (at 0 7.62) (size 1.7 1.7) (drill 1) (layers *.Cu *.Mask) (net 31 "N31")))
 (gr_line (start 85 50) (end 50 50) (layer Edge.Cuts) (width 0.15))
 (gr_line (start 85 180) (end 85 50) (layer Edge.Cuts) (width 0.15))
 (gr_line (start 50 180) (end 85 180) (layer Edge.Cuts) (width 0.15))
 (gr_line (start 50 50) (end 50 180) (layer Edge.Cuts) (width 0.15))
 (segment (start 75.75 60) (end 81.2 60) (width 0.25) (layer F.Cu) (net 3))
 (segment (start 69.2 60) (end 75.75 60) (width 0.25) (layer F.Cu) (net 3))
 (segment (start 75.75 55.55) (end 75.75 54.65) (width 0.25) (layer F.Cu) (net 3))
 (segment (start 75.75 54.65) (end 75.75 53.5) (width 0.25) (layer F.Cu) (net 3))
 (segment (start 80.2 60) (end 75.75 55.55) (width 0.25) (layer F.Cu) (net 3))
 (segment (start 81.2 60) (end 80.2 60) (width 0.25) (layer F.Cu) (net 3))
 (segment (start 74.9 51.5) (end 75.75 52.35) (width 0.25) (layer F.Cu) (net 3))
 (segment (start 72.25 51.5) (end 74.9 51.5) (width 0.25) (layer F.Cu) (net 3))
 (segment (start 75.75 52.35) (end 75.75 53.5) (width 0.25) (layer F.Cu) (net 3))
 (segment (start 70.25 53.5) (end 72.25 51.5) (width 0.25) (layer F.Cu) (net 3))
 (segment (start 62.75 53.5) (end 70.25 53.5) (width 0.25) (layer F.Cu) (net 3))
 (segment (start 75.75 67.65) (end 75.75 66.5) (width 0.25) (layer F.Cu) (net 3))
 (segment (start 74.9 68.5) (end 75.75 67.65) (width 0.25) (layer F.Cu) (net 3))
 (segment (start 72.25 68.5) (end 74.9 68.5) (width 0.25) (layer F.Cu) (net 3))
 (segment (start 70.25 66.5) (end 72.25 68.5) (width 0.25) (layer F.Cu) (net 3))
 (segment (start 62.75 66.5) (end 70.25 66.5) (width 0.25) (layer F.Cu) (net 3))
 (segment (start 75.75 64.5) (end 75.75 65.35) (width 0.25) (layer F.Cu) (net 3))
 (segment (start 75.75 65.35) (end 75.75 66.5) (width 0.25) (layer F.Cu) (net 3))
 (segment (start 80.25 60) (end 75.75 64.5) (width 0.25) (layer F.Cu) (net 3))
 (segment (start 81.2 60) (end 80.25 60) (width 0.25) (layer F.Cu) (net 3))
 (segment (start 56.45 60) (end 66.66 60) (width 0.25) (layer F.Cu) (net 4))
 (segment (start 55.6375 60) (end 56.45 60) (width 0.25) (layer F.Cu) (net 4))
 (segment (start 55.6375 66.5) (end 60.21 66.5) (width 0.25) (layer F.Cu) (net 5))
 (segment (start 55.6375 53.5) (end 60.21 53.5) (width 0.25) (layer F.Cu) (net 6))
 (segment (start 69.96 63.25) (end 73.21 66.5) (width 0.25) (layer F.Cu) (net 7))
 (segment (start 55.6375 63.25) (end 69.96 63.25) (width 0.25) (layer F.Cu) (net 7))
 (segment (start 69.96 56.75) (end 73.21 53.5) (width 0.25) (layer F.Cu) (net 8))
 (segment (start 55.6375 56.75) (end 69.96 56.75) (width 0.25) (layer F.Cu) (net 8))
 (segment (start 55.4875 109.5) (end 59.71 109.5) (width 0.25) (layer F.Cu) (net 9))
 (segment (start 69.46 112.75) (end 55.4875 112.75) (width 0.25) (layer F.Cu) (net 11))
 (segment (start 72.71 109.5) (end 69.46 112.75) (width 0.25) (layer F.Cu) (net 11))
 (segment (start 55.4875 116) (end 66.26 116) (width 0.25) (layer F.Cu) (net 12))
 (segment (start 69.46 119.25) (end 55.4875 119.25) (width 0.25) (layer F.Cu) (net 13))
 (segment (start 72.71 122.5) (end 69.46 119.25) (width 0.25) (layer F.Cu) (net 13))
 (segment (start 55.4875 122.5) (end 59.86 122.5) (width 0.25) (layer F.Cu) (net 14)))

